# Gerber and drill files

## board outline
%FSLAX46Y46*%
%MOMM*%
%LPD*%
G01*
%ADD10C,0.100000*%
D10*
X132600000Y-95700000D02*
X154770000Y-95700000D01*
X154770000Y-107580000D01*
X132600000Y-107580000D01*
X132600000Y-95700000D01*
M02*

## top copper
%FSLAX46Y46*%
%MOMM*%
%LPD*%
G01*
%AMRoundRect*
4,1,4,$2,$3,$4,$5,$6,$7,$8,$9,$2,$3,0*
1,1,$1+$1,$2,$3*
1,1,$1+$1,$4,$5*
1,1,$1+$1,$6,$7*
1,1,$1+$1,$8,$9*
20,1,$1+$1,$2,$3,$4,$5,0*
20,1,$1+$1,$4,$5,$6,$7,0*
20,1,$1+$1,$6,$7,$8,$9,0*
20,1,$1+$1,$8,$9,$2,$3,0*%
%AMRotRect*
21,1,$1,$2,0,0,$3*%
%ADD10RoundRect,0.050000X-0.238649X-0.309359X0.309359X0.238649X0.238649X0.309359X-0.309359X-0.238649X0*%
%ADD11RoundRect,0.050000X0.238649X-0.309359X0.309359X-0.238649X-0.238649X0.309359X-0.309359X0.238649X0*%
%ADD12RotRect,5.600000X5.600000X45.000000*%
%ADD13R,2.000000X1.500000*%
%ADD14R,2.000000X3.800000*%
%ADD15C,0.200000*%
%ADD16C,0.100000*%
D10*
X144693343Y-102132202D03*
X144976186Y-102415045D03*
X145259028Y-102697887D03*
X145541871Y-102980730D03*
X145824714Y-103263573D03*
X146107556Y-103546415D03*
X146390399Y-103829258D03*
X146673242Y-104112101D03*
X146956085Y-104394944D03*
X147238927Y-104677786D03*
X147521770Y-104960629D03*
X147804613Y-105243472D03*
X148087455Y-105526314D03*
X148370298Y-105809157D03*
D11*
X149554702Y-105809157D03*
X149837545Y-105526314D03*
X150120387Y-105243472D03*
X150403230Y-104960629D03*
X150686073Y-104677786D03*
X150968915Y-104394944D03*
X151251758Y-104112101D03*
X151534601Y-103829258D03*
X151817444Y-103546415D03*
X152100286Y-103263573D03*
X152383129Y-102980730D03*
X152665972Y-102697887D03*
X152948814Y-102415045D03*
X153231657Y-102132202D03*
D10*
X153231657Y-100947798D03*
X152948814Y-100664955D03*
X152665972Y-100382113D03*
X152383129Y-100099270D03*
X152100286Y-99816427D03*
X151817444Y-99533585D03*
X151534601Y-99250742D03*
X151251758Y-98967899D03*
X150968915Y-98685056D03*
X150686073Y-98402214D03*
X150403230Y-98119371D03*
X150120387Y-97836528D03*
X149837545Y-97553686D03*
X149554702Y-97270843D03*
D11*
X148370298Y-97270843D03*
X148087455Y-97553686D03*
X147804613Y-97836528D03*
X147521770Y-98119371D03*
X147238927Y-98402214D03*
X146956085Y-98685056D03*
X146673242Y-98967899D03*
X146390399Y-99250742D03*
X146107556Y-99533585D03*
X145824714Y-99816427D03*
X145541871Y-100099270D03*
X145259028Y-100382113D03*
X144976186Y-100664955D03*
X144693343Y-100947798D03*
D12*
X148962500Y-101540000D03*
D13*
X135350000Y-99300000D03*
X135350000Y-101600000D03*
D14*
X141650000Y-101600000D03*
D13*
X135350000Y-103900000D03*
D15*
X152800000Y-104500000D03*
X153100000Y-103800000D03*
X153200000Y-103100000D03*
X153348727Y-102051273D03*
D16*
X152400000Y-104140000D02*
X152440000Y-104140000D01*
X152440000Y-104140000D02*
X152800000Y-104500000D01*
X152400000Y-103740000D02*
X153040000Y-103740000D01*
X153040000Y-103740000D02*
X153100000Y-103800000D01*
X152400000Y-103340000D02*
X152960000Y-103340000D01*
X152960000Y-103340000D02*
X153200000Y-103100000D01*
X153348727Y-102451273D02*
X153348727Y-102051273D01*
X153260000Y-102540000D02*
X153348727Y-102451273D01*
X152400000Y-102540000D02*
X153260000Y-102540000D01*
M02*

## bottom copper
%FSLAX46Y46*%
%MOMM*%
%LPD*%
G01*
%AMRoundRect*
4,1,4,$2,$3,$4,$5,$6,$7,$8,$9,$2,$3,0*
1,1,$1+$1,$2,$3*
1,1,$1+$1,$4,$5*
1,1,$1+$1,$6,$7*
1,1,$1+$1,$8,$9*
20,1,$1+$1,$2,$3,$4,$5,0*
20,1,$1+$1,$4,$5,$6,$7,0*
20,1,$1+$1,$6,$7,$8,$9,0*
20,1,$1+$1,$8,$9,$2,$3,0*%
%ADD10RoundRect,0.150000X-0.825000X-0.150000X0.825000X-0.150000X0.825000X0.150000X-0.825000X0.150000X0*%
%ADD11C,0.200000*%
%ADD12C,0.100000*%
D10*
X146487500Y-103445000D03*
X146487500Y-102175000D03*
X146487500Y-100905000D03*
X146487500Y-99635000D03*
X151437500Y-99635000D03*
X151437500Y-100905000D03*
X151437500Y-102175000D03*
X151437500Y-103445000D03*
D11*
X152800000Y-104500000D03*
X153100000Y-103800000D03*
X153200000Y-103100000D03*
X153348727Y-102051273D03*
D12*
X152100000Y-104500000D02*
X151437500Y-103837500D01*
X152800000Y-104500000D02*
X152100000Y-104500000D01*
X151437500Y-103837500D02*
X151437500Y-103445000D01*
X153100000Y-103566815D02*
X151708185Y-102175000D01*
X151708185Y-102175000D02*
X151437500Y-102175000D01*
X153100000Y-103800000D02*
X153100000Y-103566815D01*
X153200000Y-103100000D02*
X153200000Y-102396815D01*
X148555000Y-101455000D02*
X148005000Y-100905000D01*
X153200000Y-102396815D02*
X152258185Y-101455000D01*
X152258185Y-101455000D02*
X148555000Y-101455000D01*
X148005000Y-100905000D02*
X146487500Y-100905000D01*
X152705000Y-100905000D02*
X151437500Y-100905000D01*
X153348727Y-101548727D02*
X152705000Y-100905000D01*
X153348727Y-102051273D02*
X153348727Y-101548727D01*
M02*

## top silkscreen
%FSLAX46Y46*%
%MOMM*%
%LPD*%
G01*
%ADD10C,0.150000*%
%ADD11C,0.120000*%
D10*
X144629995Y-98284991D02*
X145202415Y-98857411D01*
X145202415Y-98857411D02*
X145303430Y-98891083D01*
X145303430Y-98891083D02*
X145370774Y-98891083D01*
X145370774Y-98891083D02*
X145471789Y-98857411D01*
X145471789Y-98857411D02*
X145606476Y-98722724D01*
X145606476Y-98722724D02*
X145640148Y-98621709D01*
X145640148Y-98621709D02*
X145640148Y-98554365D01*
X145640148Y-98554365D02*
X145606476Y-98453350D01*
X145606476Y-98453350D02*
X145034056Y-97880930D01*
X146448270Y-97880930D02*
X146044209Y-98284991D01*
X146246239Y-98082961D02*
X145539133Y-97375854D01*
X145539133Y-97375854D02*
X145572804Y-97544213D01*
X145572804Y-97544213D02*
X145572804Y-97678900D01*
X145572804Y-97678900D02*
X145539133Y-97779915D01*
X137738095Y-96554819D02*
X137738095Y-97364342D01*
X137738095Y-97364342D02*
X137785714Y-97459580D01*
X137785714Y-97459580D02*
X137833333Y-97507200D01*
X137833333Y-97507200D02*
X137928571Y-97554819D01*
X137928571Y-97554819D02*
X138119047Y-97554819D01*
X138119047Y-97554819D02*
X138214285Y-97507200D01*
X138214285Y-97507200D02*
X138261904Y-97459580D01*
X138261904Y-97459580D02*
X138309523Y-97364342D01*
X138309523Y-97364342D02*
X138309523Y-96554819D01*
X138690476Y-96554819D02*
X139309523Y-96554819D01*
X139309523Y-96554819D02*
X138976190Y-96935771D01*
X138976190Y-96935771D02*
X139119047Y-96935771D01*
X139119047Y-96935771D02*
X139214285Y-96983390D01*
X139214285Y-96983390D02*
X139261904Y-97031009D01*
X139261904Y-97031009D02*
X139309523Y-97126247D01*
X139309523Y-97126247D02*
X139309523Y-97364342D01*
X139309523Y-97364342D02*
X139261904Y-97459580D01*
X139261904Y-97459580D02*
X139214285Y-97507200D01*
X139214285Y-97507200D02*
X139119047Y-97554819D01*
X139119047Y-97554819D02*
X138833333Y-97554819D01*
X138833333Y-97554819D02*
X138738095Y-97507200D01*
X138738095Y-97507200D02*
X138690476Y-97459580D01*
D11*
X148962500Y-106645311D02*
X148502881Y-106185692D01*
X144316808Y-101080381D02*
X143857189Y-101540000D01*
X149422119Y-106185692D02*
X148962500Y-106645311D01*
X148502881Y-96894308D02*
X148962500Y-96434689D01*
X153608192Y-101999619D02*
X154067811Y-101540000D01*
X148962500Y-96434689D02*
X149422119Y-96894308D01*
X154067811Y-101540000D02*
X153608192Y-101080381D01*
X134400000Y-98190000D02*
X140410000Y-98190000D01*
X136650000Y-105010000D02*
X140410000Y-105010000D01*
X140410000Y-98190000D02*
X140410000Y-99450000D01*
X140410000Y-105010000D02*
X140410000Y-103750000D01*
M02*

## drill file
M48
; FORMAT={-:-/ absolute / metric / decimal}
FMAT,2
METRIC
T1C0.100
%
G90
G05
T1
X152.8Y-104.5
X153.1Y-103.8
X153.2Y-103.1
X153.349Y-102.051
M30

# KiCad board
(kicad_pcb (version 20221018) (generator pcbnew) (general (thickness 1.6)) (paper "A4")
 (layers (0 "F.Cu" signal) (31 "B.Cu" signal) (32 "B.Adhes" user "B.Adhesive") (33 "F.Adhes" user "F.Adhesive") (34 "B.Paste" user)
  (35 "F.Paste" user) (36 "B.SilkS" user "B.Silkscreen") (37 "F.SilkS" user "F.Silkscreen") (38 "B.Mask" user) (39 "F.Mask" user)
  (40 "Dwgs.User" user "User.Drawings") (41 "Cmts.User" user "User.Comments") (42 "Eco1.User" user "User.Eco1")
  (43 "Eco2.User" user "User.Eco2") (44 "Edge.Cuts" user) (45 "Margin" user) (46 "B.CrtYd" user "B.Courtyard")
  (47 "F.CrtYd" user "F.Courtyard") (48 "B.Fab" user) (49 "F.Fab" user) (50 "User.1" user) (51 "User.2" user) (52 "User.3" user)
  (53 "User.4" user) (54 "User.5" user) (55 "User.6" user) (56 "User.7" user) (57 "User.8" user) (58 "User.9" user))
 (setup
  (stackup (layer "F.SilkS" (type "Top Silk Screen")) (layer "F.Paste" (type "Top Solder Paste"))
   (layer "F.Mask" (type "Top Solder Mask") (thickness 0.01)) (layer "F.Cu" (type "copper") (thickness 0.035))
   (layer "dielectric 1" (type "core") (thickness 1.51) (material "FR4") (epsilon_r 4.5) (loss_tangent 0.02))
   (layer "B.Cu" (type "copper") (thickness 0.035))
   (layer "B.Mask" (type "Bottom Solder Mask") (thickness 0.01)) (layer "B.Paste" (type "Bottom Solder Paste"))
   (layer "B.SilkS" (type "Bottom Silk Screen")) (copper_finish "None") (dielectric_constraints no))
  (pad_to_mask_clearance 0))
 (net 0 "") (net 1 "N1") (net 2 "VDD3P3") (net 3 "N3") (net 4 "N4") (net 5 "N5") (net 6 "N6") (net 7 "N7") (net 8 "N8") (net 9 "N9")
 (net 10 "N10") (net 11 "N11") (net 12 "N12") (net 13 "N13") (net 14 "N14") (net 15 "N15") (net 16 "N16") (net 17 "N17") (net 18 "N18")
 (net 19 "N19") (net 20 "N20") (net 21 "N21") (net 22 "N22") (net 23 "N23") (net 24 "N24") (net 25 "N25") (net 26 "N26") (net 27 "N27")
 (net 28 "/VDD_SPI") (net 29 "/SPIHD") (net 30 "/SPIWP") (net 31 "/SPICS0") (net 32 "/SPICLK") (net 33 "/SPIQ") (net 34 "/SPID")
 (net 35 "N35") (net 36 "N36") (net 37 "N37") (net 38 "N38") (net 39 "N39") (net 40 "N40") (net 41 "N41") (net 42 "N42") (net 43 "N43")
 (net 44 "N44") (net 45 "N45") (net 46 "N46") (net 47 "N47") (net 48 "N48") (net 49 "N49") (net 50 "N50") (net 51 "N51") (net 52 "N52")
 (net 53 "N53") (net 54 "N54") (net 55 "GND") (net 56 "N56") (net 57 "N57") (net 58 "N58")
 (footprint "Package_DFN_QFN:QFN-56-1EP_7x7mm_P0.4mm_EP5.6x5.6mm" (layer "F.Cu") (at 148.9625 101.54 45)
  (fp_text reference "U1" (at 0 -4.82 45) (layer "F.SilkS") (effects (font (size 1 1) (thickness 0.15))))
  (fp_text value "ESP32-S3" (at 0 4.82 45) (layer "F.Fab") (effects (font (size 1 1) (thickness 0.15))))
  (fp_line (start -3.61 3.61) (end -3.61 2.96) (stroke (width 0.12) (type solid)) (layer "F.SilkS"))
  (fp_line (start -2.96 -3.61) (end -3.61 -3.61) (stroke (width 0.12) (type solid)) (layer "F.SilkS"))
  (fp_line (start -2.96 3.61) (end -3.61 3.61) (stroke (width 0.12) (type solid)) (layer "F.SilkS"))
  (fp_line (start 2.96 -3.61) (end 3.61 -3.61) (stroke (width 0.12) (type solid)) (layer "F.SilkS"))
  (fp_line (start 2.96 3.61) (end 3.61 3.61) (stroke (width 0.12) (type solid)) (layer "F.SilkS"))
  (fp_line (start 3.61 -3.61) (end 3.61 -2.96) (stroke (width 0.12) (type solid)) (layer "F.SilkS"))
  (fp_line (start 3.61 3.61) (end 3.61 2.96) (stroke (width 0.12) (type solid)) (layer "F.SilkS"))
  (pad "" smd roundrect (at -2.1 -2.1 45) (size 1.13 1.13) (layers "F.Paste") (roundrect_rratio 0.221239))
  (pad "" smd roundrect (at -2.1 -0.7 45) (size 1.13 1.13) (layers "F.Paste") (roundrect_rratio 0.221239))
  (pad "" smd roundrect (at -2.1 0.7 45) (size 1.13 1.13) (layers "F.Paste") (roundrect_rratio 0.221239))
  (pad "" smd roundrect (at -2.1 2.1 45) (size 1.13 1.13) (layers "F.Paste") (roundrect_rratio 0.221239))
  (pad "" smd roundrect (at -0.7 -2.1 45) (size 1.13 1.13) (layers "F.Paste") (roundrect_rratio 0.221239))
  (pad "" smd roundrect (at -0.7 -0.7 45) (size 1.13 1.13) (layers "F.Paste") (roundrect_rratio 0.221239))
  (pad "" smd roundrect (at -0.7 0.7 45) (size 1.13 1.13) (layers "F.Paste") (roundrect_rratio 0.221239))
  (pad "" smd roundrect (at -0.7 2.1 45) (size 1.13 1.13) (layers "F.Paste") (roundrect_rratio 0.221239))
  (pad "" smd roundrect (at 0.7 -2.1 45) (size 1.13 1.13) (layers "F.Paste") (roundrect_rratio 0.221239))
  (pad "" smd roundrect (at 0.7 -0.7 45) (size 1.13 1.13) (layers "F.Paste") (roundrect_rratio 0.221239))
  (pad "" smd roundrect (at 0.7 0.7 45) (size 1.13 1.13) (layers "F.Paste") (roundrect_rratio 0.221239))
  (pad "" smd roundrect (at 0.7 2.1 45) (size 1.13 1.13) (layers "F.Paste") (roundrect_rratio 0.221239))
  (pad "" smd roundrect (at 2.1 -2.1 45) (size 1.13 1.13) (layers "F.Paste") (roundrect_rratio 0.221239))
  (pad "" smd roundrect (at 2.1 -0.7 45) (size 1.13 1.13) (layers "F.Paste") (roundrect_rratio 0.221239))
  (pad "" smd roundrect (at 2.1 0.7 45) (size 1.13 1.13) (layers "F.Paste") (roundrect_rratio 0.221239))
  (pad "" smd roundrect (at 2.1 2.1 45) (size 1.13 1.13) (layers "F.Paste") (roundrect_rratio 0.221239))
  (pad "1" smd roundrect (at -3.4375 -2.6 45) (size 0.875 0.2) (layers "F.Cu" "F.Paste" "F.Mask") (roundrect_rratio 0.25) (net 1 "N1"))
  (pad "2" smd roundrect (at -3.4375 -2.2 45) (size 0.875 0.2) (layers "F.Cu" "F.Paste" "F.Mask") (roundrect_rratio 0.25) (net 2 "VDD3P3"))
  (pad "3" smd roundrect (at -3.4375 -1.8 45) (size 0.875 0.2) (layers "F.Cu" "F.Paste" "F.Mask") (roundrect_rratio 0.25) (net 2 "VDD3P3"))
  (pad "4" smd roundrect (at -3.4375 -1.4 45) (size 0.875 0.2) (layers "F.Cu" "F.Paste" "F.Mask") (roundrect_rratio 0.25) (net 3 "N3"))
  (pad "5" smd roundrect (at -3.4375 -1 45) (size 0.875 0.2) (layers "F.Cu" "F.Paste" "F.Mask") (roundrect_rratio 0.25) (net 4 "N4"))
  (pad "6" smd roundrect (at -3.4375 -0.6 45) (size 0.875 0.2) (layers "F.Cu" "F.Paste" "F.Mask") (roundrect_rratio 0.25) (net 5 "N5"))
  (pad "7" smd roundrect (at -3.4375 -0.2 45) (size 0.875 0.2) (layers "F.Cu" "F.Paste" "F.Mask") (roundrect_rratio 0.25) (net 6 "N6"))
  (pad "8" smd roundrect (at -3.4375 0.2 45) (size 0.875 0.2) (layers "F.Cu" "F.Paste" "F.Mask") (roundrect_rratio 0.25) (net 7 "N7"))
  (pad "9" smd roundrect (at -3.4375 0.6 45) (size 0.875 0.2) (layers "F.Cu" "F.Paste" "F.Mask") (roundrect_rratio 0.25) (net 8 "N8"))
  (pad "10" smd roundrect (at -3.4375 1 45) (size 0.875 0.2) (layers "F.Cu" "F.Paste" "F.Mask") (roundrect_rratio 0.25) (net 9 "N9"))
  (pad "11" smd roundrect (at -3.4375 1.4 45) (size 0.875 0.2) (layers "F.Cu" "F.Paste" "F.Mask") (roundrect_rratio 0.25) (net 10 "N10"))
  (pad "12" smd roundrect (at -3.4375 1.8 45) (size 0.875 0.2) (layers "F.Cu" "F.Paste" "F.Mask") (roundrect_rratio 0.25) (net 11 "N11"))
  (pad "13" smd roundrect (at -3.4375 2.2 45) (size 0.875 0.2) (layers "F.Cu" "F.Paste" "F.Mask") (roundrect_rratio 0.25) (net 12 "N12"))
  (pad "14" smd roundrect (at -3.4375 2.6 45) (size 0.875 0.2) (layers "F.Cu" "F.Paste" "F.Mask") (roundrect_rratio 0.25) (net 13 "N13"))
  (pad "15" smd roundrect (at -2.6 3.4375 45) (size 0.2 0.875) (layers "F.Cu" "F.Paste" "F.Mask") (roundrect_rratio 0.25) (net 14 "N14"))
  (pad "16" smd roundrect (at -2.2 3.4375 45) (size 0.2 0.875) (layers "F.Cu" "F.Paste" "F.Mask") (roundrect_rratio 0.25) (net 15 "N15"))
  (pad "17" smd roundrect (at -1.8 3.4375 45) (size 0.2 0.875) (layers "F.Cu" "F.Paste" "F.Mask") (roundrect_rratio 0.25) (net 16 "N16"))
  (pad "18" smd roundrect (at -1.4 3.4375 45) (size 0.2 0.875) (layers "F.Cu" "F.Paste" "F.Mask") (roundrect_rratio 0.25) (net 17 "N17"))
  (pad "19" smd roundrect (at -1 3.4375 45) (size 0.2 0.875) (layers "F.Cu" "F.Paste" "F.Mask") (roundrect_rratio 0.25) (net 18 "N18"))
  (pad "20" smd roundrect (at -0.6 3.4375 45) (size 0.2 0.875) (layers "F.Cu" "F.Paste" "F.Mask") (roundrect_rratio 0.25) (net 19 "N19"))
  (pad "21" smd roundrect (at -0.2 3.4375 45) (size 0.2 0.875) (layers "F.Cu" "F.Paste" "F.Mask") (roundrect_rratio 0.25) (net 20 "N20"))
  (pad "22" smd roundrect (at 0.2 3.4375 45) (size 0.2 0.875) (layers "F.Cu" "F.Paste" "F.Mask") (roundrect_rratio 0.25) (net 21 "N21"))
  (pad "23" smd roundrect (at 0.6 3.4375 45) (size 0.2 0.875) (layers "F.Cu" "F.Paste" "F.Mask") (roundrect_rratio 0.25) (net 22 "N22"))
  (pad "24" smd roundrect (at 1 3.4375 45) (size 0.2 0.875) (layers "F.Cu" "F.Paste" "F.Mask") (roundrect_rratio 0.25) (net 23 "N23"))
  (pad "25" smd roundrect (at 1.4 3.4375 45) (size 0.2 0.875) (layers "F.Cu" "F.Paste" "F.Mask") (roundrect_rratio 0.25) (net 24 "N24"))
  (pad "26" smd roundrect (at 1.8 3.4375 45) (size 0.2 0.875) (layers "F.Cu" "F.Paste" "F.Mask") (roundrect_rratio 0.25) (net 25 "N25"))
  (pad "27" smd roundrect (at 2.2 3.4375 45) (size 0.2 0.875) (layers "F.Cu" "F.Paste" "F.Mask") (roundrect_rratio 0.25) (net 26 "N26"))
  (pad "28" smd roundrect (at 2.6 3.4375 45) (size 0.2 0.875) (layers "F.Cu" "F.Paste" "F.Mask") (roundrect_rratio 0.25) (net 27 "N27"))
  (pad "29" smd roundrect (at 3.4375 2.6 45) (size 0.875 0.2) (layers "F.Cu" "F.Paste" "F.Mask") (roundrect_rratio 0.25) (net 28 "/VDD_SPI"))
  (pad "30" smd roundrect (at 3.4375 2.2 45) (size 0.875 0.2) (layers "F.Cu" "F.Paste" "F.Mask") (roundrect_rratio 0.25) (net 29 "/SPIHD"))
  (pad "31" smd roundrect (at 3.4375 1.8 45) (size 0.875 0.2) (layers "F.Cu" "F.Paste" "F.Mask") (roundrect_rratio 0.25) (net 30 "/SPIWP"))
  (pad "32" smd roundrect (at 3.4375 1.4 45) (size 0.875 0.2) (layers "F.Cu" "F.Paste" "F.Mask") (roundrect_rratio 0.25) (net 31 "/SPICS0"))
  (pad "33" smd roundrect (at 3.4375 1 45) (size 0.875 0.2) (layers "F.Cu" "F.Paste" "F.Mask") (roundrect_rratio 0.25) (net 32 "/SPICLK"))
  (pad "34" smd roundrect (at 3.4375 0.6 45) (size 0.875 0.2) (layers "F.Cu" "F.Paste" "F.Mask") (roundrect_rratio 0.25) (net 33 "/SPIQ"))
  (pad "35" smd roundrect (at 3.4375 0.2 45) (size 0.875 0.2) (layers "F.Cu" "F.Paste" "F.Mask") (roundrect_rratio 0.25) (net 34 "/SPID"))
  (pad "36" smd roundrect (at 3.4375 -0.2 45) (size 0.875 0.2) (layers "F.Cu" "F.Paste" "F.Mask") (roundrect_rratio 0.25) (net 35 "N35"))
  (pad "37" smd roundrect (at 3.4375 -0.6 45) (size 0.875 0.2) (layers "F.Cu" "F.Paste" "F.Mask") (roundrect_rratio 0.25) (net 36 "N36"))
  (pad "38" smd roundrect (at 3.4375 -1 45) (size 0.875 0.2) (layers "F.Cu" "F.Paste" "F.Mask") (roundrect_rratio 0.25) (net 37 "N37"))
  (pad "39" smd roundrect (at 3.4375 -1.4 45) (size 0.875 0.2) (layers "F.Cu" "F.Paste" "F.Mask") (roundrect_rratio 0.25) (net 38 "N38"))
  (pad "40" smd roundrect (at 3.4375 -1.8 45) (size 0.875 0.2) (layers "F.Cu" "F.Paste" "F.Mask") (roundrect_rratio 0.25) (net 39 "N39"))
  (pad "41" smd roundrect (at 3.4375 -2.2 45) (size 0.875 0.2) (layers "F.Cu" "F.Paste" "F.Mask") (roundrect_rratio 0.25) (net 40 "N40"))
  (pad "42" smd roundrect (at 3.4375 -2.6 45) (size 0.875 0.2) (layers "F.Cu" "F.Paste" "F.Mask") (roundrect_rratio 0.25) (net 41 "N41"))
  (pad "43" smd roundrect (at 2.6 -3.4375 45) (size 0.2 0.875) (layers "F.Cu" "F.Paste" "F.Mask") (roundrect_rratio 0.25) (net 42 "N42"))
  (pad "44" smd roundrect (at 2.2 -3.4375 45) (size 0.2 0.875) (layers "F.Cu" "F.Paste" "F.Mask") (roundrect_rratio 0.25) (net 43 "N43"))
  (pad "45" smd roundrect (at 1.8 -3.4375 45) (size 0.2 0.875) (layers "F.Cu" "F.Paste" "F.Mask") (roundrect_rratio 0.25) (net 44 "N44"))
  (pad "46" smd roundrect (at 1.4 -3.4375 45) (size 0.2 0.875) (layers "F.Cu" "F.Paste" "F.Mask") (roundrect_rratio 0.25) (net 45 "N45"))
  (pad "47" smd roundrect (at 1 -3.4375 45) (size 0.2 0.875) (layers "F.Cu" "F.Paste" "F.Mask") (roundrect_rratio 0.25) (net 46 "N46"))
  (pad "48" smd roundrect (at 0.6 -3.4375 45) (size 0.2 0.875) (layers "F.Cu" "F.Paste" "F.Mask") (roundrect_rratio 0.25) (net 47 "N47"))
  (pad "49" smd roundrect (at 0.2 -3.4375 45) (size 0.2 0.875) (layers "F.Cu" "F.Paste" "F.Mask") (roundrect_rratio 0.25) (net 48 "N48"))
  (pad "50" smd roundrect (at -0.2 -3.4375 45) (size 0.2 0.875) (layers "F.Cu" "F.Paste" "F.Mask") (roundrect_rratio 0.25) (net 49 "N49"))
  (pad "51" smd roundrect (at -0.6 -3.4375 45) (size 0.2 0.875) (layers "F.Cu" "F.Paste" "F.Mask") (roundrect_rratio 0.25) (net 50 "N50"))
  (pad "52" smd roundrect (at -1 -3.4375 45) (size 0.2 0.875) (layers "F.Cu" "F.Paste" "F.Mask") (roundrect_rratio 0.25) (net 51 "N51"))
  (pad "53" smd roundrect (at -1.4 -3.4375 45) (size 0.2 0.875) (layers "F.Cu" "F.Paste" "F.Mask") (roundrect_rratio 0.25) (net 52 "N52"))
  (pad "54" smd roundrect (at -1.8 -3.4375 45) (size 0.2 0.875) (layers "F.Cu" "F.Paste" "F.Mask") (roundrect_rratio 0.25) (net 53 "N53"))
  (pad "55" smd roundrect (at -2.2 -3.4375 45) (size 0.2 0.875) (layers "F.Cu" "F.Paste" "F.Mask") (roundrect_rratio 0.25) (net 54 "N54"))
  (pad "56" smd roundrect (at -2.6 -3.4375 45) (size 0.2 0.875) (layers "F.Cu" "F.Paste" "F.Mask") (roundrect_rratio 0.25) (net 54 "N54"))
  (pad "57" smd rect (at 0 0 45) (size 5.6 5.6) (layers "F.Cu" "F.Mask") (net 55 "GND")))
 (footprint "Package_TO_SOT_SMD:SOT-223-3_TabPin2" (layer "F.Cu") (at 138.5 101.6)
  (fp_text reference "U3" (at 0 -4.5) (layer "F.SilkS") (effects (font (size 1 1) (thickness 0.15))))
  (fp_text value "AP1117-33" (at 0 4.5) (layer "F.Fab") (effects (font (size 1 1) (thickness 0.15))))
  (fp_line (start -4.1 -3.41) (end 1.91 -3.41) (stroke (width 0.12) (type solid)) (layer "F.SilkS"))
  (fp_line (start -1.85 3.41) (end 1.91 3.41) (stroke (width 0.12) (type solid)) (layer "F.SilkS"))
  (fp_line (start 1.91 -3.41) (end 1.91 -2.15) (stroke (width 0.12) (type solid)) (layer "F.SilkS"))
  (fp_line (start 1.91 3.41) (end 1.91 2.15) (stroke (width 0.12) (type solid)) (layer "F.SilkS"))
  (pad "1" smd rect (at -3.15 -2.3) (size 2 1.5) (layers "F.Cu" "F.Paste" "F.Mask") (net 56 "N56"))
  (pad "2" smd rect (at -3.15 0) (size 2 1.5) (layers "F.Cu" "F.Paste" "F.Mask") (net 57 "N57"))
  (pad "2" smd rect (at 3.15 0) (size 2 3.8) (layers "F.Cu" "F.Paste" "F.Mask") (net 57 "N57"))
  (pad "3" smd rect (at -3.15 2.3) (size 2 1.5) (layers "F.Cu" "F.Paste" "F.Mask") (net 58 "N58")))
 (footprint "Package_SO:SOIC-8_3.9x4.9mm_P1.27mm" (layer "B.Cu") (at 148.9625 101.54)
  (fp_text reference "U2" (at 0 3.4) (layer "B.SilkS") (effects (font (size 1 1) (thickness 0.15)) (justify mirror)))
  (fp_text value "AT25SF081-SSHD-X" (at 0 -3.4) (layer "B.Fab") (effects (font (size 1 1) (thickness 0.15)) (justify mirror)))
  (pad "1" smd roundrect (at -2.475 1.905) (size 1.95 0.6) (layers "B.Cu" "B.Paste" "B.Mask") (roundrect_rratio 0.25) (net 31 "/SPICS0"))
  (pad "2" smd roundrect (at -2.475 0.635) (size 1.95 0.6) (layers "B.Cu" "B.Paste" "B.Mask") (roundrect_rratio 0.25) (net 33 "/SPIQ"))
  (pad "3" smd roundrect (at -2.475 -0.635) (size 1.95 0.6) (layers "B.Cu" "B.Paste" "B.Mask") (roundrect_rratio 0.25) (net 30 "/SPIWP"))
  (pad "4" smd roundrect (at -2.475 -1.905) (size 1.95 0.6) (layers "B.Cu" "B.Paste" "B.Mask") (roundrect_rratio 0.25) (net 55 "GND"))
  (pad "5" smd roundrect (at 2.475 -1.905) (size 1.95 0.6) (layers "B.Cu" "B.Paste" "B.Mask") (roundrect_rratio 0.25) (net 34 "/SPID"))
  (pad "6" smd roundrect (at 2.475 -0.635) (size 1.95 0.6) (layers "B.Cu" "B.Paste" "B.Mask") (roundrect_rratio 0.25) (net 32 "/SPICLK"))
  (pad "7" smd roundrect (at 2.475 0.635) (size 1.95 0.6) (layers "B.Cu" "B.Paste" "B.Mask") (roundrect_rratio 0.25) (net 29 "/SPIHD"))
  (pad "8" smd roundrect (at 2.475 1.905) (size 1.95 0.6) (layers "B.Cu" "B.Paste" "B.Mask") (roundrect_rratio 0.25) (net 28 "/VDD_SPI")))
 (gr_rect (start 132.6 95.7) (end 154.77 107.58) (stroke (width 0.1) (type default)) (fill none) (layer "Edge.Cuts"))
 (segment (start 152.4 104.14) (end 152.44 104.14) (width 0.1) (layer "F.Cu") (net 28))
 (segment (start 152.44 104.14) (end 152.8 104.5) (width 0.1) (layer "F.Cu") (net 28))
 (via (at 152.8 104.5) (size 0.2) (drill 0.1) (layers "F.Cu" "B.Cu") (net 28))
 (segment (start 152.1 104.5) (end 151.4375 103.8375) (width 0.1) (layer "B.Cu") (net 28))
 (segment (start 152.8 104.5) (end 152.1 104.5) (width 0.1) (layer "B.Cu") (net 28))
 (segment (start 151.4375 103.8375) (end 151.4375 103.445) (width 0.1) (layer "B.Cu") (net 28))
 (segment (start 152.4 103.74) (end 153.04 103.74) (width 0.1) (layer "F.Cu") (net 29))
 (segment (start 153.04 103.74) (end 153.1 103.8) (width 0.1) (layer "F.Cu") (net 29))
 (via (at 153.1 103.8) (size 0.2) (drill 0.1) (layers "F.Cu" "B.Cu") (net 29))
 (segment (start 153.1 103.566815) (end 151.708185 102.175) (width 0.1) (layer "B.Cu") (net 29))
 (segment (start 151.708185 102.175) (end 151.4375 102.175) (width 0.1) (layer "B.Cu") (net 29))
 (segment (start 153.1 103.8) (end 153.1 103.566815) (width 0.1) (layer "B.Cu") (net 29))
 (segment (start 152.4 103.34) (end 152.96 103.34) (width 0.1) (layer "F.Cu") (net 30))
 (segment (start 152.96 103.34) (end 153.2 103.1) (width 0.1) (layer "F.Cu") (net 30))
 (via (at 153.2 103.1) (size 0.2) (drill 0.1) (layers "F.Cu" "B.Cu") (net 30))
 (segment (start 153.2 103.1) (end 153.2 102.396815) (width 0.1) (layer "B.Cu") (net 30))
 (segment (start 148.555 101.455) (end 148.005 100.905) (width 0.1) (layer "B.Cu") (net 30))
 (segment (start 153.2 102.396815) (end 152.258185 101.455) (width 0.1) (layer "B.Cu") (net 30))
 (segment (start 152.258185 101.455) (end 148.555 101.455) (width 0.1) (layer "B.Cu") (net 30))
 (segment (start 148.005 100.905) (end 146.4875 100.905) (width 0.1) (layer "B.Cu") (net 30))
 (segment (start 153.348727 102.451273) (end 153.348727 102.051273) (width 0.1) (layer "F.Cu") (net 32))
 (segment (start 153.26 102.54) (end 153.348727 102.451273) (width 0.1) (layer "F.Cu") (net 32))
 (segment (start 152.4 102.54) (end 153.26 102.54) (width 0.1) (layer "F.Cu") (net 32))
 (via (at 153.348727 102.051273) (size 0.2) (drill 0.1) (layers "F.Cu" "B.Cu") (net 32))
 (segment (start 152.705 100.905) (end 151.4375 100.905) (width 0.1) (layer "B.Cu") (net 32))
 (segment (start 153.348727 101.548727) (end 152.705 100.905) (width 0.1) (layer "B.Cu") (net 32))
 (segment (start 153.348727 102.051273) (end 153.348727 101.548727) (width 0.1) (layer "B.Cu") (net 32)))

